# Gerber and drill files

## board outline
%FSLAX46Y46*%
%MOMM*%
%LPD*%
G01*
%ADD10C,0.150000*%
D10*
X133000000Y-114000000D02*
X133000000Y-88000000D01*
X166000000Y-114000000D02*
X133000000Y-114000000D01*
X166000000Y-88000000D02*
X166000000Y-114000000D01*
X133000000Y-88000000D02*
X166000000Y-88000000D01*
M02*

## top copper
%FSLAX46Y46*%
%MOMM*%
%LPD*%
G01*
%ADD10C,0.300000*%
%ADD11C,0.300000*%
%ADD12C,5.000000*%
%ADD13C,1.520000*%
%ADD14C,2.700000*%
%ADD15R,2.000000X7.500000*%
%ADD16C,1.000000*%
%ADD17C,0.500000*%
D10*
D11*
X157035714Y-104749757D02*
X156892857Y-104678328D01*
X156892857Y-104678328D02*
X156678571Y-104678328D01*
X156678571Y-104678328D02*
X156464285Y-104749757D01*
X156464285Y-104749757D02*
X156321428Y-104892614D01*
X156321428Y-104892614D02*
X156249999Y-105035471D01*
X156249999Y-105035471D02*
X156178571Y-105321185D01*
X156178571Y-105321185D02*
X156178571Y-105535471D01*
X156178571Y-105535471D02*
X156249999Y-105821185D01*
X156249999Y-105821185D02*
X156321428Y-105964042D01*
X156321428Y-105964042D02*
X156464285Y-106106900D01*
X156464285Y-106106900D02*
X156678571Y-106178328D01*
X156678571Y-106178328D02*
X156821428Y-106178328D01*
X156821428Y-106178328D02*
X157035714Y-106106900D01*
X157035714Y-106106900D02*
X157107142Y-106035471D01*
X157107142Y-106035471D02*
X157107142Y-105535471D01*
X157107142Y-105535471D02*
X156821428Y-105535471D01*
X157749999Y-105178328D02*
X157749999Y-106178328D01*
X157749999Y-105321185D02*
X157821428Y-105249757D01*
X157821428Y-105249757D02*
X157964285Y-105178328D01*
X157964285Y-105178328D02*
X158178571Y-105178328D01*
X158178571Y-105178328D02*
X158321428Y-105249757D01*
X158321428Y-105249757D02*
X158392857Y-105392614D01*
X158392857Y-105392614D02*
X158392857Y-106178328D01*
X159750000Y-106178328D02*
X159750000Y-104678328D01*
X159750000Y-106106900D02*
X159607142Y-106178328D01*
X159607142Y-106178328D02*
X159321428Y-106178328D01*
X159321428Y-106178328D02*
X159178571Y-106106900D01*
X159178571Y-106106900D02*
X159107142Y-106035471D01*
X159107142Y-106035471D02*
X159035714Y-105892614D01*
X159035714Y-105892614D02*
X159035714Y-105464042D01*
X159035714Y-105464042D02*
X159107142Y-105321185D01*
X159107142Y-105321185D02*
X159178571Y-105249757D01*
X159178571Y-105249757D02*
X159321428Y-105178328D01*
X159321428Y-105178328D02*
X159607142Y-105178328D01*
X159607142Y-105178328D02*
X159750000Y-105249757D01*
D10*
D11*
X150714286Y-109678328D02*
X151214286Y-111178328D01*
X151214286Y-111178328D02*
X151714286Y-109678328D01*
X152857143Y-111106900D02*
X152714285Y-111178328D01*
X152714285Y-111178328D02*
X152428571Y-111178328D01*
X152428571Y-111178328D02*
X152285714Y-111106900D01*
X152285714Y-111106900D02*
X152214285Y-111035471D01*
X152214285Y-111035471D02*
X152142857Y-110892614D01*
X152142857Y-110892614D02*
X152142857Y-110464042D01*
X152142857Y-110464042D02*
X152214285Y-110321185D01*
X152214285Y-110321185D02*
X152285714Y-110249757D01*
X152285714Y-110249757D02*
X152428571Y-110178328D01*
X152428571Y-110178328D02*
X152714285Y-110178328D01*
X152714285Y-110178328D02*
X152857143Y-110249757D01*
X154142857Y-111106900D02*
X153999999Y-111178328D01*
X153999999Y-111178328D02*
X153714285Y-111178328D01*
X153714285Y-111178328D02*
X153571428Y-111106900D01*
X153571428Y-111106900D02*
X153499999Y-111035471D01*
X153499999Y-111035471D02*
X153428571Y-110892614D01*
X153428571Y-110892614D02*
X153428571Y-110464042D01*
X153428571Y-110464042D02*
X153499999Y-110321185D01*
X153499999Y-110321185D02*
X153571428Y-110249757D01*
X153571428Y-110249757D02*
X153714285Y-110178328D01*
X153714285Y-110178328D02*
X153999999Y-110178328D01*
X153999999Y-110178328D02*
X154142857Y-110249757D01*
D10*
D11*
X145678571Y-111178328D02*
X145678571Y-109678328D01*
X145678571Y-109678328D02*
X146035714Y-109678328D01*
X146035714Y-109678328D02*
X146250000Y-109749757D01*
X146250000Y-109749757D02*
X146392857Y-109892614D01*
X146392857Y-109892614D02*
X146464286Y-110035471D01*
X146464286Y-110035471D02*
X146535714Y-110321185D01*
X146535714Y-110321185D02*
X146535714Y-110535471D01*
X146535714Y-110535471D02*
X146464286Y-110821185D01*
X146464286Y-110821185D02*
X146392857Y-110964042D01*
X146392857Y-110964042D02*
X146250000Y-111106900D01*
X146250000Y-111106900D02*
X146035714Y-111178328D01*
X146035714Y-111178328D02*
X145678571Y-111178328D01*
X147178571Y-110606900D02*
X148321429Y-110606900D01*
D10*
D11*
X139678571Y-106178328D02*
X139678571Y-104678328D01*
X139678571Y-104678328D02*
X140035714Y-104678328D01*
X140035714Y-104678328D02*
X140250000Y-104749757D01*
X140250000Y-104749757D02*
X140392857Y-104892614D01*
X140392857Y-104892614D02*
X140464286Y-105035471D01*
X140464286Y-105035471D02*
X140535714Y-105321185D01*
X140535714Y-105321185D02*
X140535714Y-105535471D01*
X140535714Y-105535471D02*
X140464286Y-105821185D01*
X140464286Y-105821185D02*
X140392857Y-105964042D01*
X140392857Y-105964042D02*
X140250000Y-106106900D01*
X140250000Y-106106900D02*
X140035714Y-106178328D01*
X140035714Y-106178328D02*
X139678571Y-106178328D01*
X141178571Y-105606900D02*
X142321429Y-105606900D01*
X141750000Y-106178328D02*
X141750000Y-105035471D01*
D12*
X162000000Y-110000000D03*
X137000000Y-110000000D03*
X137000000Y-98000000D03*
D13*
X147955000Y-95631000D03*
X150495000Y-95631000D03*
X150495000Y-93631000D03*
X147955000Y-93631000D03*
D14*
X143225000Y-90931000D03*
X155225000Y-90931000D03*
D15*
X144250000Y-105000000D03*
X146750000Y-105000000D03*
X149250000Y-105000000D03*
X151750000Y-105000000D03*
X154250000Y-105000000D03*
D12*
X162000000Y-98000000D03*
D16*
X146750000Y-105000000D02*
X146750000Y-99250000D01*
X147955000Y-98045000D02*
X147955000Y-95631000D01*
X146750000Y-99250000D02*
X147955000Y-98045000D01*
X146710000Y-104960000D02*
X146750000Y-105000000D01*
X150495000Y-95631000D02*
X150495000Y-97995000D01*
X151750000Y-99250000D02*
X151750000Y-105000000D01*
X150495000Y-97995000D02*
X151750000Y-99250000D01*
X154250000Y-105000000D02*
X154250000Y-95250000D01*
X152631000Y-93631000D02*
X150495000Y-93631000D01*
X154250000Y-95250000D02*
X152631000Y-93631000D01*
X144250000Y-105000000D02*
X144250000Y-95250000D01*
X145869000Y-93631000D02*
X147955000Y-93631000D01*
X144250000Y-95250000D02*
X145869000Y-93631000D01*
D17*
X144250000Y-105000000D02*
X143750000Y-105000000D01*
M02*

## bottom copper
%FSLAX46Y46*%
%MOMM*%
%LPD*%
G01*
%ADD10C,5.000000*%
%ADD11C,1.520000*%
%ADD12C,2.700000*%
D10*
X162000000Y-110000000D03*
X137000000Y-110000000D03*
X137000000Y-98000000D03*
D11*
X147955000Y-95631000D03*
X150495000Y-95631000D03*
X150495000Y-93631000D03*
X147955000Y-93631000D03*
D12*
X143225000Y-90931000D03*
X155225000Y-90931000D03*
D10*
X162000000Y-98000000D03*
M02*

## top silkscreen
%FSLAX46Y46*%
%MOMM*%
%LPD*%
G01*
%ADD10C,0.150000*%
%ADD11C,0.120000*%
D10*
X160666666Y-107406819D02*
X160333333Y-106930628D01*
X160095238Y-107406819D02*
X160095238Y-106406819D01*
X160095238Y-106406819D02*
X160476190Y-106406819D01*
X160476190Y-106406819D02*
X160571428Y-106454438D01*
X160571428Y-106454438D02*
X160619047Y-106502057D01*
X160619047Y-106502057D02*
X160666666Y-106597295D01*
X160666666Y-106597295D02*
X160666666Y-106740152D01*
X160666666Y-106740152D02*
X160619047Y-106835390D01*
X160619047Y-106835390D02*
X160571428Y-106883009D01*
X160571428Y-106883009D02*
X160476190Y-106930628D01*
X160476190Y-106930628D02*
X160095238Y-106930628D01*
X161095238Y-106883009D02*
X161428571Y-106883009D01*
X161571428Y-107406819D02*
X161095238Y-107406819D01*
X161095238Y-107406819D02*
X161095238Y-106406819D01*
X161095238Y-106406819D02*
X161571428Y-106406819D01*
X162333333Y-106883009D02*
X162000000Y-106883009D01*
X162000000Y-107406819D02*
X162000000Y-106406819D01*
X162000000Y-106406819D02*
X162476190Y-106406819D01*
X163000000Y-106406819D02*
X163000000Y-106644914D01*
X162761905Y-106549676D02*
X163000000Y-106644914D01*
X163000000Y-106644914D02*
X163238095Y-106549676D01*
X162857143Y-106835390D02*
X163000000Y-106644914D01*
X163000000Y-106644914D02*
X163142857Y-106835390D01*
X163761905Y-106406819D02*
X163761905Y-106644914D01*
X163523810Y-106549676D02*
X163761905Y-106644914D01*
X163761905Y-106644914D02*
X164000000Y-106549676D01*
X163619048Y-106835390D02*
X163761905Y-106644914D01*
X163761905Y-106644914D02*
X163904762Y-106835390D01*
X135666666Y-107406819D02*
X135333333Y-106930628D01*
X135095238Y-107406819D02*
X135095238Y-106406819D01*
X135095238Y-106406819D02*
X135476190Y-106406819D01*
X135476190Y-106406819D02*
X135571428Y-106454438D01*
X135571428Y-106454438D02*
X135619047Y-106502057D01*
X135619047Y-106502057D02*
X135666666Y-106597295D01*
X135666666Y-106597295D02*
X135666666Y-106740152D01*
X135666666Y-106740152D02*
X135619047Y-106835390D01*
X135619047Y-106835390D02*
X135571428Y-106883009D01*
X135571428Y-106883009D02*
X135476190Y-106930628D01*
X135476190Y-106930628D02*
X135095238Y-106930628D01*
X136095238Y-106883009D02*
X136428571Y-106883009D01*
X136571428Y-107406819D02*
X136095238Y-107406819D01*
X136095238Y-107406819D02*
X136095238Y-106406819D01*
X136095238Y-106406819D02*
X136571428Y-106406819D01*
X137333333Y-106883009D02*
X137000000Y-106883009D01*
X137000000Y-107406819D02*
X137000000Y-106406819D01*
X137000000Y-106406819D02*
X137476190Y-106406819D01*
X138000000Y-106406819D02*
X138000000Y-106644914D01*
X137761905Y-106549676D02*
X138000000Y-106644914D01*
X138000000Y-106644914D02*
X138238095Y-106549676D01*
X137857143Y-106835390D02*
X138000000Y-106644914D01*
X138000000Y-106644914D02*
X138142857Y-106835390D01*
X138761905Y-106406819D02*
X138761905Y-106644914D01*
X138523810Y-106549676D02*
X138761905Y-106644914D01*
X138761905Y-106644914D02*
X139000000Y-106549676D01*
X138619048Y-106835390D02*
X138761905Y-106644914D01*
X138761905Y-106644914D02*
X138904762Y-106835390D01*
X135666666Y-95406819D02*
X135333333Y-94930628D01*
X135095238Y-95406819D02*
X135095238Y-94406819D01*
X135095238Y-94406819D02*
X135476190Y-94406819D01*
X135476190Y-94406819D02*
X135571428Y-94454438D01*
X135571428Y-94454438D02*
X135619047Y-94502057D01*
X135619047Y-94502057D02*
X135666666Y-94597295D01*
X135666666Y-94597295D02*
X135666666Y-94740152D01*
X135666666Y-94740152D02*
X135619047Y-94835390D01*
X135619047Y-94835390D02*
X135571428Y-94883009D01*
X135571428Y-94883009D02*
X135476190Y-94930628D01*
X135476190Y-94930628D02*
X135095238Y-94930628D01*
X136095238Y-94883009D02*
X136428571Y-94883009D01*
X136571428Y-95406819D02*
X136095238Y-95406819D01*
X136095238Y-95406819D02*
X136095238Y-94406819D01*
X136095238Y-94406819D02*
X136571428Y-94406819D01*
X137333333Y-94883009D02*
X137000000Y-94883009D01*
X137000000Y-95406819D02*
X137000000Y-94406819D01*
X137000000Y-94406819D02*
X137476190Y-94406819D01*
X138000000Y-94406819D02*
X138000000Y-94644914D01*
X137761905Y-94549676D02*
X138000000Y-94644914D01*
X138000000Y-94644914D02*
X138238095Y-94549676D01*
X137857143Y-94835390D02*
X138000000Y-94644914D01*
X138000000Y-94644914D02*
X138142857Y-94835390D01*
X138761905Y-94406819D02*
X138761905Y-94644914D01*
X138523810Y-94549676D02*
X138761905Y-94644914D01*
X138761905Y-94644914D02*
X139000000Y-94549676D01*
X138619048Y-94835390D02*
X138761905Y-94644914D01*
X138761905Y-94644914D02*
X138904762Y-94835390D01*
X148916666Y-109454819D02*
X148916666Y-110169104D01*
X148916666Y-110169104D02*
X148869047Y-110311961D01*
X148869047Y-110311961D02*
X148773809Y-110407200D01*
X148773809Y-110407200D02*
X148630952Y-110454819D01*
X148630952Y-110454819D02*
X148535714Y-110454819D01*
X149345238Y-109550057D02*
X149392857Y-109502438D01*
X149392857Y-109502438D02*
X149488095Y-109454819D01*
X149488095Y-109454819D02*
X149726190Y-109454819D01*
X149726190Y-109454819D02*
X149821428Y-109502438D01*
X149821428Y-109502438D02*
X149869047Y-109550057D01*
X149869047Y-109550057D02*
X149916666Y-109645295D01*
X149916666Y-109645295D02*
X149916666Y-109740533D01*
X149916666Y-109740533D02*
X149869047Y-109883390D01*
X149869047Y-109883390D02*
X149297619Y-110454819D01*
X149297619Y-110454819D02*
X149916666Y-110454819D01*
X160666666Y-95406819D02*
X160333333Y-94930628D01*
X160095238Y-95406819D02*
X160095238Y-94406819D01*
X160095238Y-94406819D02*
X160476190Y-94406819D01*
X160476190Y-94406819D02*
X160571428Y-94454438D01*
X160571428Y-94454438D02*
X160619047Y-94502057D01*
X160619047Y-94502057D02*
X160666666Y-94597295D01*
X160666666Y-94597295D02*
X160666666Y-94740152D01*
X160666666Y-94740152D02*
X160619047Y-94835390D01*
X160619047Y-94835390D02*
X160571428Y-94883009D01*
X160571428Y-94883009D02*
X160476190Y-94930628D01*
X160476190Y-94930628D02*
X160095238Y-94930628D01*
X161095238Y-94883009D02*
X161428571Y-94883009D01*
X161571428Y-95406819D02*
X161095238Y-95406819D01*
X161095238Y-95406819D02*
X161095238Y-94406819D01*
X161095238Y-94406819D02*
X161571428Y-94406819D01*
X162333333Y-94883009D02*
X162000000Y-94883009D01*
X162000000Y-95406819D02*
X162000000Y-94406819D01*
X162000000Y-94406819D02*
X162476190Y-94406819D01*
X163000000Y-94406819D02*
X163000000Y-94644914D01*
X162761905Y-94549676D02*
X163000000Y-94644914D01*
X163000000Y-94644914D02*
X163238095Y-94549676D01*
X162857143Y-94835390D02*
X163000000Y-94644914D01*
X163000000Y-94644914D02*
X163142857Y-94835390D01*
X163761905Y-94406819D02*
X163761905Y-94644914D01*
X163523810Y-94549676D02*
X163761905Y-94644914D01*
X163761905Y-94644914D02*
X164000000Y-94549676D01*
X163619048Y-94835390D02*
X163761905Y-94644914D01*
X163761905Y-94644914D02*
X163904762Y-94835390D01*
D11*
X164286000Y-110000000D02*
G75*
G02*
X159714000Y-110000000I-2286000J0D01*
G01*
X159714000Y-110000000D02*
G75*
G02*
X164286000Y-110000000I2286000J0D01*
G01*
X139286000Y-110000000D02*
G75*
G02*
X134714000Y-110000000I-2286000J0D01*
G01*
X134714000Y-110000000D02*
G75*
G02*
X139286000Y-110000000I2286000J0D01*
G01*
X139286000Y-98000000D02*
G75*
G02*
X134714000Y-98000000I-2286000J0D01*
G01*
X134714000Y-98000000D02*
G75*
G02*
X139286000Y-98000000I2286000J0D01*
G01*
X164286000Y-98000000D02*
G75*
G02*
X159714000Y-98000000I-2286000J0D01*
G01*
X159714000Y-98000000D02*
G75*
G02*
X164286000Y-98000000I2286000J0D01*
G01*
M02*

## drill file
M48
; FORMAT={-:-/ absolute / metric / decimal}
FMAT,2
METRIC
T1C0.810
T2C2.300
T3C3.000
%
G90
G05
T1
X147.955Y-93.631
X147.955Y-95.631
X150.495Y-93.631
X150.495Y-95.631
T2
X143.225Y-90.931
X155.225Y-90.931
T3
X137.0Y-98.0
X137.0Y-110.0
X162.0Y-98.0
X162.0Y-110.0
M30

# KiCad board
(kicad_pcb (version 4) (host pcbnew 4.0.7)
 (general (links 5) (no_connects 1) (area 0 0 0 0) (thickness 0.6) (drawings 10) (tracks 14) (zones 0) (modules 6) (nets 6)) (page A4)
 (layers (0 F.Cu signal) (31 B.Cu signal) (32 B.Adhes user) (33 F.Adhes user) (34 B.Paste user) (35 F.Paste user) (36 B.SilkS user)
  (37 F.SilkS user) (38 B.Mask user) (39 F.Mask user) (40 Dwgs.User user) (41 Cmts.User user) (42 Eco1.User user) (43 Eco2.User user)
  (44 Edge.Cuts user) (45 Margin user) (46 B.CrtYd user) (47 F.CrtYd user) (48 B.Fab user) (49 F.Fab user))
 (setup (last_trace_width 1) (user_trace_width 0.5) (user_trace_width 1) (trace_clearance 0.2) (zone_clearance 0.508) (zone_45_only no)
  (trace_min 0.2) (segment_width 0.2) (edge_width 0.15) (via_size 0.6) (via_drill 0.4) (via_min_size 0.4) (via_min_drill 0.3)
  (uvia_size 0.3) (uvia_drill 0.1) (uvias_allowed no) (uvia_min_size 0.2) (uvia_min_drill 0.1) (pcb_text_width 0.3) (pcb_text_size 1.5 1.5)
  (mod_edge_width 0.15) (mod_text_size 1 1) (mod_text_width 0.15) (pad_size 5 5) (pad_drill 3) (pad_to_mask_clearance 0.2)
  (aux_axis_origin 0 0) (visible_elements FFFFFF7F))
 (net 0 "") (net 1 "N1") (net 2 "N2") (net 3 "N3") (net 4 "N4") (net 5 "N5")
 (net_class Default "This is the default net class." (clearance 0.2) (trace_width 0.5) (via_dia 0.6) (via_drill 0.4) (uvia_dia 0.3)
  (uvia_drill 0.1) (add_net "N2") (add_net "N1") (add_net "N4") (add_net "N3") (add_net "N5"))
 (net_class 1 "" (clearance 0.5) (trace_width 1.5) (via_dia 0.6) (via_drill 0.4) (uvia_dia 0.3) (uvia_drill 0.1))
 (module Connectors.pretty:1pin (layer F.Cu) (at 162 110)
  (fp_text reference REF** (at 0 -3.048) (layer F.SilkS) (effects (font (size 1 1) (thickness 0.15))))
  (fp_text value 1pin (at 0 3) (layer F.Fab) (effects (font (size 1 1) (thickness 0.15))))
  (fp_circle (center 0 0) (end 0 -2.286) (layer F.SilkS) (width 0.12))
  (pad 1 thru_hole circle (at 0 0) (size 5 5) (drill 3) (layers *.Cu *.Mask)))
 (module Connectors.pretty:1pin (layer F.Cu) (at 137 110)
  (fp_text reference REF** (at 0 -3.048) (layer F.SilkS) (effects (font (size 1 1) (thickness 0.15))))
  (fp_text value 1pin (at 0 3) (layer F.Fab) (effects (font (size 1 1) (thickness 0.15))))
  (fp_circle (center 0 0) (end 0 -2.286) (layer F.SilkS) (width 0.12))
  (pad 1 thru_hole circle (at 0 0) (size 5 5) (drill 3) (layers *.Cu *.Mask)))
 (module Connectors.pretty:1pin (layer F.Cu) (at 137 98)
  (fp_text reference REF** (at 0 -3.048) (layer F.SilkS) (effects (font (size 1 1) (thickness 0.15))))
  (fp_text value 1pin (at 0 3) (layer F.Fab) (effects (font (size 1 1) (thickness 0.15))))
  (fp_circle (center 0 0) (end 0 -2.286) (layer F.SilkS) (width 0.12))
  (pad 1 thru_hole circle (at 0 0) (size 5 5) (drill 3) (layers *.Cu *.Mask)))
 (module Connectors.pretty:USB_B (layer B.Cu) (at 150.495 95.631 90)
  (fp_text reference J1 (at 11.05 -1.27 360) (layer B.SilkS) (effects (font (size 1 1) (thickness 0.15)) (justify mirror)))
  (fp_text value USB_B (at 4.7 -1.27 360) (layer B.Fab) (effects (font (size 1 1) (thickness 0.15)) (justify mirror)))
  (pad 2 thru_hole circle (at 0 -2.54 180) (size 1.52 1.52) (drill 0.81) (layers *.Cu *.Mask) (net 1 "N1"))
  (pad 1 thru_hole circle (at 0 0 180) (size 1.52 1.52) (drill 0.81) (layers *.Cu *.Mask) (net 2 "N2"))
  (pad 4 thru_hole circle (at 2 0 180) (size 1.52 1.52) (drill 0.81) (layers *.Cu *.Mask) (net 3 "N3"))
  (pad 3 thru_hole circle (at 2 -2.54 180) (size 1.52 1.52) (drill 0.81) (layers *.Cu *.Mask) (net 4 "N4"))
  (pad 5 thru_hole circle (at 4.7 -7.27 180) (size 2.7 2.7) (drill 2.3) (layers *.Cu *.Mask) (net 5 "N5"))
  (pad 5 thru_hole circle (at 4.7 4.73 180) (size 2.7 2.7) (drill 2.3) (layers *.Cu *.Mask) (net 5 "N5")))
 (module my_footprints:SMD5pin (layer F.Cu) (at 149.25 105)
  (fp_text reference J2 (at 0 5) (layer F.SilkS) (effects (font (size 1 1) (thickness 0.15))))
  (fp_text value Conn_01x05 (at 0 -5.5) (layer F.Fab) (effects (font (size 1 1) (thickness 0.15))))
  (pad 1 smd rect (at -5 0) (size 2 7.5) (layers F.Cu F.Paste F.Mask) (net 4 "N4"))
  (pad 2 smd rect (at -2.5 0) (size 2 7.5) (layers F.Cu F.Paste F.Mask) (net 1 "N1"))
  (pad 3 smd rect (at 0 0) (size 2 7.5) (layers F.Cu F.Paste F.Mask))
  (pad 4 smd rect (at 2.5 0) (size 2 7.5) (layers F.Cu F.Paste F.Mask) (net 2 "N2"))
  (pad 5 smd rect (at 5 0) (size 2 7.5) (layers F.Cu F.Paste F.Mask) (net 3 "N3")))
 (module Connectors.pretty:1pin (layer F.Cu) (at 162 98)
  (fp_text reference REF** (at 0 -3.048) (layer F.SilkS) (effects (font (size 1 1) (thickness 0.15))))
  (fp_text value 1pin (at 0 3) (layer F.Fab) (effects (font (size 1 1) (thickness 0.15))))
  (fp_circle (center 0 0) (end 0 -2.286) (layer F.SilkS) (width 0.12))
  (pad 1 thru_hole circle (at 0 0) (size 5 5) (drill 3) (layers *.Cu *.Mask)))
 (gr_line (start 133 114) (end 133 88) (angle 90) (layer Edge.Cuts) (width 0.15))
 (gr_line (start 166 114) (end 133 114) (angle 90) (layer Edge.Cuts) (width 0.15))
 (gr_line (start 166 88) (end 166 114) (angle 90) (layer Edge.Cuts) (width 0.15))
 (gr_line (start 133 88) (end 166 88) (angle 90) (layer Edge.Cuts) (width 0.15))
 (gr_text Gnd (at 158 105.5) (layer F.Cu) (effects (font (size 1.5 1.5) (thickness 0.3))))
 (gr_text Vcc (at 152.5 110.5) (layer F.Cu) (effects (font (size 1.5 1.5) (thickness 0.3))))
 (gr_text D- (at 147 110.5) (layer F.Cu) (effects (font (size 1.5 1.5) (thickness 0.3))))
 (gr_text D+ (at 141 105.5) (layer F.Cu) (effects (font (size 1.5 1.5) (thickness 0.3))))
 (segment (start 146.75 105) (end 146.75 99.25) (width 1) (layer F.Cu) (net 1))
 (segment (start 147.955 98.045) (end 147.955 95.631) (width 1) (layer F.Cu) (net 1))
 (segment (start 146.75 99.25) (end 147.955 98.045) (width 1) (layer F.Cu) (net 1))
 (segment (start 146.71 104.96) (end 146.75 105) (width 1) (layer F.Cu) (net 1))
 (segment (start 150.495 95.631) (end 150.495 97.995) (width 1) (layer F.Cu) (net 2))
 (segment (start 151.75 99.25) (end 151.75 105) (width 1) (layer F.Cu) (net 2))
 (segment (start 150.495 97.995) (end 151.75 99.25) (width 1) (layer F.Cu) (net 2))
 (segment (start 154.25 105) (end 154.25 95.25) (width 1) (layer F.Cu) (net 3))
 (segment (start 152.631 93.631) (end 150.495 93.631) (width 1) (layer F.Cu) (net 3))
 (segment (start 154.25 95.25) (end 152.631 93.631) (width 1) (layer F.Cu) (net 3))
 (segment (start 144.25 105) (end 144.25 95.25) (width 1) (layer F.Cu) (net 4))
 (segment (start 145.869 93.631) (end 147.955 93.631) (width 1) (layer F.Cu) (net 4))
 (segment (start 144.25 95.25) (end 145.869 93.631) (width 1) (layer F.Cu) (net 4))
 (segment (start 144.25 105) (end 143.75 105) (width 0.5) (layer F.Cu) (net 4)))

